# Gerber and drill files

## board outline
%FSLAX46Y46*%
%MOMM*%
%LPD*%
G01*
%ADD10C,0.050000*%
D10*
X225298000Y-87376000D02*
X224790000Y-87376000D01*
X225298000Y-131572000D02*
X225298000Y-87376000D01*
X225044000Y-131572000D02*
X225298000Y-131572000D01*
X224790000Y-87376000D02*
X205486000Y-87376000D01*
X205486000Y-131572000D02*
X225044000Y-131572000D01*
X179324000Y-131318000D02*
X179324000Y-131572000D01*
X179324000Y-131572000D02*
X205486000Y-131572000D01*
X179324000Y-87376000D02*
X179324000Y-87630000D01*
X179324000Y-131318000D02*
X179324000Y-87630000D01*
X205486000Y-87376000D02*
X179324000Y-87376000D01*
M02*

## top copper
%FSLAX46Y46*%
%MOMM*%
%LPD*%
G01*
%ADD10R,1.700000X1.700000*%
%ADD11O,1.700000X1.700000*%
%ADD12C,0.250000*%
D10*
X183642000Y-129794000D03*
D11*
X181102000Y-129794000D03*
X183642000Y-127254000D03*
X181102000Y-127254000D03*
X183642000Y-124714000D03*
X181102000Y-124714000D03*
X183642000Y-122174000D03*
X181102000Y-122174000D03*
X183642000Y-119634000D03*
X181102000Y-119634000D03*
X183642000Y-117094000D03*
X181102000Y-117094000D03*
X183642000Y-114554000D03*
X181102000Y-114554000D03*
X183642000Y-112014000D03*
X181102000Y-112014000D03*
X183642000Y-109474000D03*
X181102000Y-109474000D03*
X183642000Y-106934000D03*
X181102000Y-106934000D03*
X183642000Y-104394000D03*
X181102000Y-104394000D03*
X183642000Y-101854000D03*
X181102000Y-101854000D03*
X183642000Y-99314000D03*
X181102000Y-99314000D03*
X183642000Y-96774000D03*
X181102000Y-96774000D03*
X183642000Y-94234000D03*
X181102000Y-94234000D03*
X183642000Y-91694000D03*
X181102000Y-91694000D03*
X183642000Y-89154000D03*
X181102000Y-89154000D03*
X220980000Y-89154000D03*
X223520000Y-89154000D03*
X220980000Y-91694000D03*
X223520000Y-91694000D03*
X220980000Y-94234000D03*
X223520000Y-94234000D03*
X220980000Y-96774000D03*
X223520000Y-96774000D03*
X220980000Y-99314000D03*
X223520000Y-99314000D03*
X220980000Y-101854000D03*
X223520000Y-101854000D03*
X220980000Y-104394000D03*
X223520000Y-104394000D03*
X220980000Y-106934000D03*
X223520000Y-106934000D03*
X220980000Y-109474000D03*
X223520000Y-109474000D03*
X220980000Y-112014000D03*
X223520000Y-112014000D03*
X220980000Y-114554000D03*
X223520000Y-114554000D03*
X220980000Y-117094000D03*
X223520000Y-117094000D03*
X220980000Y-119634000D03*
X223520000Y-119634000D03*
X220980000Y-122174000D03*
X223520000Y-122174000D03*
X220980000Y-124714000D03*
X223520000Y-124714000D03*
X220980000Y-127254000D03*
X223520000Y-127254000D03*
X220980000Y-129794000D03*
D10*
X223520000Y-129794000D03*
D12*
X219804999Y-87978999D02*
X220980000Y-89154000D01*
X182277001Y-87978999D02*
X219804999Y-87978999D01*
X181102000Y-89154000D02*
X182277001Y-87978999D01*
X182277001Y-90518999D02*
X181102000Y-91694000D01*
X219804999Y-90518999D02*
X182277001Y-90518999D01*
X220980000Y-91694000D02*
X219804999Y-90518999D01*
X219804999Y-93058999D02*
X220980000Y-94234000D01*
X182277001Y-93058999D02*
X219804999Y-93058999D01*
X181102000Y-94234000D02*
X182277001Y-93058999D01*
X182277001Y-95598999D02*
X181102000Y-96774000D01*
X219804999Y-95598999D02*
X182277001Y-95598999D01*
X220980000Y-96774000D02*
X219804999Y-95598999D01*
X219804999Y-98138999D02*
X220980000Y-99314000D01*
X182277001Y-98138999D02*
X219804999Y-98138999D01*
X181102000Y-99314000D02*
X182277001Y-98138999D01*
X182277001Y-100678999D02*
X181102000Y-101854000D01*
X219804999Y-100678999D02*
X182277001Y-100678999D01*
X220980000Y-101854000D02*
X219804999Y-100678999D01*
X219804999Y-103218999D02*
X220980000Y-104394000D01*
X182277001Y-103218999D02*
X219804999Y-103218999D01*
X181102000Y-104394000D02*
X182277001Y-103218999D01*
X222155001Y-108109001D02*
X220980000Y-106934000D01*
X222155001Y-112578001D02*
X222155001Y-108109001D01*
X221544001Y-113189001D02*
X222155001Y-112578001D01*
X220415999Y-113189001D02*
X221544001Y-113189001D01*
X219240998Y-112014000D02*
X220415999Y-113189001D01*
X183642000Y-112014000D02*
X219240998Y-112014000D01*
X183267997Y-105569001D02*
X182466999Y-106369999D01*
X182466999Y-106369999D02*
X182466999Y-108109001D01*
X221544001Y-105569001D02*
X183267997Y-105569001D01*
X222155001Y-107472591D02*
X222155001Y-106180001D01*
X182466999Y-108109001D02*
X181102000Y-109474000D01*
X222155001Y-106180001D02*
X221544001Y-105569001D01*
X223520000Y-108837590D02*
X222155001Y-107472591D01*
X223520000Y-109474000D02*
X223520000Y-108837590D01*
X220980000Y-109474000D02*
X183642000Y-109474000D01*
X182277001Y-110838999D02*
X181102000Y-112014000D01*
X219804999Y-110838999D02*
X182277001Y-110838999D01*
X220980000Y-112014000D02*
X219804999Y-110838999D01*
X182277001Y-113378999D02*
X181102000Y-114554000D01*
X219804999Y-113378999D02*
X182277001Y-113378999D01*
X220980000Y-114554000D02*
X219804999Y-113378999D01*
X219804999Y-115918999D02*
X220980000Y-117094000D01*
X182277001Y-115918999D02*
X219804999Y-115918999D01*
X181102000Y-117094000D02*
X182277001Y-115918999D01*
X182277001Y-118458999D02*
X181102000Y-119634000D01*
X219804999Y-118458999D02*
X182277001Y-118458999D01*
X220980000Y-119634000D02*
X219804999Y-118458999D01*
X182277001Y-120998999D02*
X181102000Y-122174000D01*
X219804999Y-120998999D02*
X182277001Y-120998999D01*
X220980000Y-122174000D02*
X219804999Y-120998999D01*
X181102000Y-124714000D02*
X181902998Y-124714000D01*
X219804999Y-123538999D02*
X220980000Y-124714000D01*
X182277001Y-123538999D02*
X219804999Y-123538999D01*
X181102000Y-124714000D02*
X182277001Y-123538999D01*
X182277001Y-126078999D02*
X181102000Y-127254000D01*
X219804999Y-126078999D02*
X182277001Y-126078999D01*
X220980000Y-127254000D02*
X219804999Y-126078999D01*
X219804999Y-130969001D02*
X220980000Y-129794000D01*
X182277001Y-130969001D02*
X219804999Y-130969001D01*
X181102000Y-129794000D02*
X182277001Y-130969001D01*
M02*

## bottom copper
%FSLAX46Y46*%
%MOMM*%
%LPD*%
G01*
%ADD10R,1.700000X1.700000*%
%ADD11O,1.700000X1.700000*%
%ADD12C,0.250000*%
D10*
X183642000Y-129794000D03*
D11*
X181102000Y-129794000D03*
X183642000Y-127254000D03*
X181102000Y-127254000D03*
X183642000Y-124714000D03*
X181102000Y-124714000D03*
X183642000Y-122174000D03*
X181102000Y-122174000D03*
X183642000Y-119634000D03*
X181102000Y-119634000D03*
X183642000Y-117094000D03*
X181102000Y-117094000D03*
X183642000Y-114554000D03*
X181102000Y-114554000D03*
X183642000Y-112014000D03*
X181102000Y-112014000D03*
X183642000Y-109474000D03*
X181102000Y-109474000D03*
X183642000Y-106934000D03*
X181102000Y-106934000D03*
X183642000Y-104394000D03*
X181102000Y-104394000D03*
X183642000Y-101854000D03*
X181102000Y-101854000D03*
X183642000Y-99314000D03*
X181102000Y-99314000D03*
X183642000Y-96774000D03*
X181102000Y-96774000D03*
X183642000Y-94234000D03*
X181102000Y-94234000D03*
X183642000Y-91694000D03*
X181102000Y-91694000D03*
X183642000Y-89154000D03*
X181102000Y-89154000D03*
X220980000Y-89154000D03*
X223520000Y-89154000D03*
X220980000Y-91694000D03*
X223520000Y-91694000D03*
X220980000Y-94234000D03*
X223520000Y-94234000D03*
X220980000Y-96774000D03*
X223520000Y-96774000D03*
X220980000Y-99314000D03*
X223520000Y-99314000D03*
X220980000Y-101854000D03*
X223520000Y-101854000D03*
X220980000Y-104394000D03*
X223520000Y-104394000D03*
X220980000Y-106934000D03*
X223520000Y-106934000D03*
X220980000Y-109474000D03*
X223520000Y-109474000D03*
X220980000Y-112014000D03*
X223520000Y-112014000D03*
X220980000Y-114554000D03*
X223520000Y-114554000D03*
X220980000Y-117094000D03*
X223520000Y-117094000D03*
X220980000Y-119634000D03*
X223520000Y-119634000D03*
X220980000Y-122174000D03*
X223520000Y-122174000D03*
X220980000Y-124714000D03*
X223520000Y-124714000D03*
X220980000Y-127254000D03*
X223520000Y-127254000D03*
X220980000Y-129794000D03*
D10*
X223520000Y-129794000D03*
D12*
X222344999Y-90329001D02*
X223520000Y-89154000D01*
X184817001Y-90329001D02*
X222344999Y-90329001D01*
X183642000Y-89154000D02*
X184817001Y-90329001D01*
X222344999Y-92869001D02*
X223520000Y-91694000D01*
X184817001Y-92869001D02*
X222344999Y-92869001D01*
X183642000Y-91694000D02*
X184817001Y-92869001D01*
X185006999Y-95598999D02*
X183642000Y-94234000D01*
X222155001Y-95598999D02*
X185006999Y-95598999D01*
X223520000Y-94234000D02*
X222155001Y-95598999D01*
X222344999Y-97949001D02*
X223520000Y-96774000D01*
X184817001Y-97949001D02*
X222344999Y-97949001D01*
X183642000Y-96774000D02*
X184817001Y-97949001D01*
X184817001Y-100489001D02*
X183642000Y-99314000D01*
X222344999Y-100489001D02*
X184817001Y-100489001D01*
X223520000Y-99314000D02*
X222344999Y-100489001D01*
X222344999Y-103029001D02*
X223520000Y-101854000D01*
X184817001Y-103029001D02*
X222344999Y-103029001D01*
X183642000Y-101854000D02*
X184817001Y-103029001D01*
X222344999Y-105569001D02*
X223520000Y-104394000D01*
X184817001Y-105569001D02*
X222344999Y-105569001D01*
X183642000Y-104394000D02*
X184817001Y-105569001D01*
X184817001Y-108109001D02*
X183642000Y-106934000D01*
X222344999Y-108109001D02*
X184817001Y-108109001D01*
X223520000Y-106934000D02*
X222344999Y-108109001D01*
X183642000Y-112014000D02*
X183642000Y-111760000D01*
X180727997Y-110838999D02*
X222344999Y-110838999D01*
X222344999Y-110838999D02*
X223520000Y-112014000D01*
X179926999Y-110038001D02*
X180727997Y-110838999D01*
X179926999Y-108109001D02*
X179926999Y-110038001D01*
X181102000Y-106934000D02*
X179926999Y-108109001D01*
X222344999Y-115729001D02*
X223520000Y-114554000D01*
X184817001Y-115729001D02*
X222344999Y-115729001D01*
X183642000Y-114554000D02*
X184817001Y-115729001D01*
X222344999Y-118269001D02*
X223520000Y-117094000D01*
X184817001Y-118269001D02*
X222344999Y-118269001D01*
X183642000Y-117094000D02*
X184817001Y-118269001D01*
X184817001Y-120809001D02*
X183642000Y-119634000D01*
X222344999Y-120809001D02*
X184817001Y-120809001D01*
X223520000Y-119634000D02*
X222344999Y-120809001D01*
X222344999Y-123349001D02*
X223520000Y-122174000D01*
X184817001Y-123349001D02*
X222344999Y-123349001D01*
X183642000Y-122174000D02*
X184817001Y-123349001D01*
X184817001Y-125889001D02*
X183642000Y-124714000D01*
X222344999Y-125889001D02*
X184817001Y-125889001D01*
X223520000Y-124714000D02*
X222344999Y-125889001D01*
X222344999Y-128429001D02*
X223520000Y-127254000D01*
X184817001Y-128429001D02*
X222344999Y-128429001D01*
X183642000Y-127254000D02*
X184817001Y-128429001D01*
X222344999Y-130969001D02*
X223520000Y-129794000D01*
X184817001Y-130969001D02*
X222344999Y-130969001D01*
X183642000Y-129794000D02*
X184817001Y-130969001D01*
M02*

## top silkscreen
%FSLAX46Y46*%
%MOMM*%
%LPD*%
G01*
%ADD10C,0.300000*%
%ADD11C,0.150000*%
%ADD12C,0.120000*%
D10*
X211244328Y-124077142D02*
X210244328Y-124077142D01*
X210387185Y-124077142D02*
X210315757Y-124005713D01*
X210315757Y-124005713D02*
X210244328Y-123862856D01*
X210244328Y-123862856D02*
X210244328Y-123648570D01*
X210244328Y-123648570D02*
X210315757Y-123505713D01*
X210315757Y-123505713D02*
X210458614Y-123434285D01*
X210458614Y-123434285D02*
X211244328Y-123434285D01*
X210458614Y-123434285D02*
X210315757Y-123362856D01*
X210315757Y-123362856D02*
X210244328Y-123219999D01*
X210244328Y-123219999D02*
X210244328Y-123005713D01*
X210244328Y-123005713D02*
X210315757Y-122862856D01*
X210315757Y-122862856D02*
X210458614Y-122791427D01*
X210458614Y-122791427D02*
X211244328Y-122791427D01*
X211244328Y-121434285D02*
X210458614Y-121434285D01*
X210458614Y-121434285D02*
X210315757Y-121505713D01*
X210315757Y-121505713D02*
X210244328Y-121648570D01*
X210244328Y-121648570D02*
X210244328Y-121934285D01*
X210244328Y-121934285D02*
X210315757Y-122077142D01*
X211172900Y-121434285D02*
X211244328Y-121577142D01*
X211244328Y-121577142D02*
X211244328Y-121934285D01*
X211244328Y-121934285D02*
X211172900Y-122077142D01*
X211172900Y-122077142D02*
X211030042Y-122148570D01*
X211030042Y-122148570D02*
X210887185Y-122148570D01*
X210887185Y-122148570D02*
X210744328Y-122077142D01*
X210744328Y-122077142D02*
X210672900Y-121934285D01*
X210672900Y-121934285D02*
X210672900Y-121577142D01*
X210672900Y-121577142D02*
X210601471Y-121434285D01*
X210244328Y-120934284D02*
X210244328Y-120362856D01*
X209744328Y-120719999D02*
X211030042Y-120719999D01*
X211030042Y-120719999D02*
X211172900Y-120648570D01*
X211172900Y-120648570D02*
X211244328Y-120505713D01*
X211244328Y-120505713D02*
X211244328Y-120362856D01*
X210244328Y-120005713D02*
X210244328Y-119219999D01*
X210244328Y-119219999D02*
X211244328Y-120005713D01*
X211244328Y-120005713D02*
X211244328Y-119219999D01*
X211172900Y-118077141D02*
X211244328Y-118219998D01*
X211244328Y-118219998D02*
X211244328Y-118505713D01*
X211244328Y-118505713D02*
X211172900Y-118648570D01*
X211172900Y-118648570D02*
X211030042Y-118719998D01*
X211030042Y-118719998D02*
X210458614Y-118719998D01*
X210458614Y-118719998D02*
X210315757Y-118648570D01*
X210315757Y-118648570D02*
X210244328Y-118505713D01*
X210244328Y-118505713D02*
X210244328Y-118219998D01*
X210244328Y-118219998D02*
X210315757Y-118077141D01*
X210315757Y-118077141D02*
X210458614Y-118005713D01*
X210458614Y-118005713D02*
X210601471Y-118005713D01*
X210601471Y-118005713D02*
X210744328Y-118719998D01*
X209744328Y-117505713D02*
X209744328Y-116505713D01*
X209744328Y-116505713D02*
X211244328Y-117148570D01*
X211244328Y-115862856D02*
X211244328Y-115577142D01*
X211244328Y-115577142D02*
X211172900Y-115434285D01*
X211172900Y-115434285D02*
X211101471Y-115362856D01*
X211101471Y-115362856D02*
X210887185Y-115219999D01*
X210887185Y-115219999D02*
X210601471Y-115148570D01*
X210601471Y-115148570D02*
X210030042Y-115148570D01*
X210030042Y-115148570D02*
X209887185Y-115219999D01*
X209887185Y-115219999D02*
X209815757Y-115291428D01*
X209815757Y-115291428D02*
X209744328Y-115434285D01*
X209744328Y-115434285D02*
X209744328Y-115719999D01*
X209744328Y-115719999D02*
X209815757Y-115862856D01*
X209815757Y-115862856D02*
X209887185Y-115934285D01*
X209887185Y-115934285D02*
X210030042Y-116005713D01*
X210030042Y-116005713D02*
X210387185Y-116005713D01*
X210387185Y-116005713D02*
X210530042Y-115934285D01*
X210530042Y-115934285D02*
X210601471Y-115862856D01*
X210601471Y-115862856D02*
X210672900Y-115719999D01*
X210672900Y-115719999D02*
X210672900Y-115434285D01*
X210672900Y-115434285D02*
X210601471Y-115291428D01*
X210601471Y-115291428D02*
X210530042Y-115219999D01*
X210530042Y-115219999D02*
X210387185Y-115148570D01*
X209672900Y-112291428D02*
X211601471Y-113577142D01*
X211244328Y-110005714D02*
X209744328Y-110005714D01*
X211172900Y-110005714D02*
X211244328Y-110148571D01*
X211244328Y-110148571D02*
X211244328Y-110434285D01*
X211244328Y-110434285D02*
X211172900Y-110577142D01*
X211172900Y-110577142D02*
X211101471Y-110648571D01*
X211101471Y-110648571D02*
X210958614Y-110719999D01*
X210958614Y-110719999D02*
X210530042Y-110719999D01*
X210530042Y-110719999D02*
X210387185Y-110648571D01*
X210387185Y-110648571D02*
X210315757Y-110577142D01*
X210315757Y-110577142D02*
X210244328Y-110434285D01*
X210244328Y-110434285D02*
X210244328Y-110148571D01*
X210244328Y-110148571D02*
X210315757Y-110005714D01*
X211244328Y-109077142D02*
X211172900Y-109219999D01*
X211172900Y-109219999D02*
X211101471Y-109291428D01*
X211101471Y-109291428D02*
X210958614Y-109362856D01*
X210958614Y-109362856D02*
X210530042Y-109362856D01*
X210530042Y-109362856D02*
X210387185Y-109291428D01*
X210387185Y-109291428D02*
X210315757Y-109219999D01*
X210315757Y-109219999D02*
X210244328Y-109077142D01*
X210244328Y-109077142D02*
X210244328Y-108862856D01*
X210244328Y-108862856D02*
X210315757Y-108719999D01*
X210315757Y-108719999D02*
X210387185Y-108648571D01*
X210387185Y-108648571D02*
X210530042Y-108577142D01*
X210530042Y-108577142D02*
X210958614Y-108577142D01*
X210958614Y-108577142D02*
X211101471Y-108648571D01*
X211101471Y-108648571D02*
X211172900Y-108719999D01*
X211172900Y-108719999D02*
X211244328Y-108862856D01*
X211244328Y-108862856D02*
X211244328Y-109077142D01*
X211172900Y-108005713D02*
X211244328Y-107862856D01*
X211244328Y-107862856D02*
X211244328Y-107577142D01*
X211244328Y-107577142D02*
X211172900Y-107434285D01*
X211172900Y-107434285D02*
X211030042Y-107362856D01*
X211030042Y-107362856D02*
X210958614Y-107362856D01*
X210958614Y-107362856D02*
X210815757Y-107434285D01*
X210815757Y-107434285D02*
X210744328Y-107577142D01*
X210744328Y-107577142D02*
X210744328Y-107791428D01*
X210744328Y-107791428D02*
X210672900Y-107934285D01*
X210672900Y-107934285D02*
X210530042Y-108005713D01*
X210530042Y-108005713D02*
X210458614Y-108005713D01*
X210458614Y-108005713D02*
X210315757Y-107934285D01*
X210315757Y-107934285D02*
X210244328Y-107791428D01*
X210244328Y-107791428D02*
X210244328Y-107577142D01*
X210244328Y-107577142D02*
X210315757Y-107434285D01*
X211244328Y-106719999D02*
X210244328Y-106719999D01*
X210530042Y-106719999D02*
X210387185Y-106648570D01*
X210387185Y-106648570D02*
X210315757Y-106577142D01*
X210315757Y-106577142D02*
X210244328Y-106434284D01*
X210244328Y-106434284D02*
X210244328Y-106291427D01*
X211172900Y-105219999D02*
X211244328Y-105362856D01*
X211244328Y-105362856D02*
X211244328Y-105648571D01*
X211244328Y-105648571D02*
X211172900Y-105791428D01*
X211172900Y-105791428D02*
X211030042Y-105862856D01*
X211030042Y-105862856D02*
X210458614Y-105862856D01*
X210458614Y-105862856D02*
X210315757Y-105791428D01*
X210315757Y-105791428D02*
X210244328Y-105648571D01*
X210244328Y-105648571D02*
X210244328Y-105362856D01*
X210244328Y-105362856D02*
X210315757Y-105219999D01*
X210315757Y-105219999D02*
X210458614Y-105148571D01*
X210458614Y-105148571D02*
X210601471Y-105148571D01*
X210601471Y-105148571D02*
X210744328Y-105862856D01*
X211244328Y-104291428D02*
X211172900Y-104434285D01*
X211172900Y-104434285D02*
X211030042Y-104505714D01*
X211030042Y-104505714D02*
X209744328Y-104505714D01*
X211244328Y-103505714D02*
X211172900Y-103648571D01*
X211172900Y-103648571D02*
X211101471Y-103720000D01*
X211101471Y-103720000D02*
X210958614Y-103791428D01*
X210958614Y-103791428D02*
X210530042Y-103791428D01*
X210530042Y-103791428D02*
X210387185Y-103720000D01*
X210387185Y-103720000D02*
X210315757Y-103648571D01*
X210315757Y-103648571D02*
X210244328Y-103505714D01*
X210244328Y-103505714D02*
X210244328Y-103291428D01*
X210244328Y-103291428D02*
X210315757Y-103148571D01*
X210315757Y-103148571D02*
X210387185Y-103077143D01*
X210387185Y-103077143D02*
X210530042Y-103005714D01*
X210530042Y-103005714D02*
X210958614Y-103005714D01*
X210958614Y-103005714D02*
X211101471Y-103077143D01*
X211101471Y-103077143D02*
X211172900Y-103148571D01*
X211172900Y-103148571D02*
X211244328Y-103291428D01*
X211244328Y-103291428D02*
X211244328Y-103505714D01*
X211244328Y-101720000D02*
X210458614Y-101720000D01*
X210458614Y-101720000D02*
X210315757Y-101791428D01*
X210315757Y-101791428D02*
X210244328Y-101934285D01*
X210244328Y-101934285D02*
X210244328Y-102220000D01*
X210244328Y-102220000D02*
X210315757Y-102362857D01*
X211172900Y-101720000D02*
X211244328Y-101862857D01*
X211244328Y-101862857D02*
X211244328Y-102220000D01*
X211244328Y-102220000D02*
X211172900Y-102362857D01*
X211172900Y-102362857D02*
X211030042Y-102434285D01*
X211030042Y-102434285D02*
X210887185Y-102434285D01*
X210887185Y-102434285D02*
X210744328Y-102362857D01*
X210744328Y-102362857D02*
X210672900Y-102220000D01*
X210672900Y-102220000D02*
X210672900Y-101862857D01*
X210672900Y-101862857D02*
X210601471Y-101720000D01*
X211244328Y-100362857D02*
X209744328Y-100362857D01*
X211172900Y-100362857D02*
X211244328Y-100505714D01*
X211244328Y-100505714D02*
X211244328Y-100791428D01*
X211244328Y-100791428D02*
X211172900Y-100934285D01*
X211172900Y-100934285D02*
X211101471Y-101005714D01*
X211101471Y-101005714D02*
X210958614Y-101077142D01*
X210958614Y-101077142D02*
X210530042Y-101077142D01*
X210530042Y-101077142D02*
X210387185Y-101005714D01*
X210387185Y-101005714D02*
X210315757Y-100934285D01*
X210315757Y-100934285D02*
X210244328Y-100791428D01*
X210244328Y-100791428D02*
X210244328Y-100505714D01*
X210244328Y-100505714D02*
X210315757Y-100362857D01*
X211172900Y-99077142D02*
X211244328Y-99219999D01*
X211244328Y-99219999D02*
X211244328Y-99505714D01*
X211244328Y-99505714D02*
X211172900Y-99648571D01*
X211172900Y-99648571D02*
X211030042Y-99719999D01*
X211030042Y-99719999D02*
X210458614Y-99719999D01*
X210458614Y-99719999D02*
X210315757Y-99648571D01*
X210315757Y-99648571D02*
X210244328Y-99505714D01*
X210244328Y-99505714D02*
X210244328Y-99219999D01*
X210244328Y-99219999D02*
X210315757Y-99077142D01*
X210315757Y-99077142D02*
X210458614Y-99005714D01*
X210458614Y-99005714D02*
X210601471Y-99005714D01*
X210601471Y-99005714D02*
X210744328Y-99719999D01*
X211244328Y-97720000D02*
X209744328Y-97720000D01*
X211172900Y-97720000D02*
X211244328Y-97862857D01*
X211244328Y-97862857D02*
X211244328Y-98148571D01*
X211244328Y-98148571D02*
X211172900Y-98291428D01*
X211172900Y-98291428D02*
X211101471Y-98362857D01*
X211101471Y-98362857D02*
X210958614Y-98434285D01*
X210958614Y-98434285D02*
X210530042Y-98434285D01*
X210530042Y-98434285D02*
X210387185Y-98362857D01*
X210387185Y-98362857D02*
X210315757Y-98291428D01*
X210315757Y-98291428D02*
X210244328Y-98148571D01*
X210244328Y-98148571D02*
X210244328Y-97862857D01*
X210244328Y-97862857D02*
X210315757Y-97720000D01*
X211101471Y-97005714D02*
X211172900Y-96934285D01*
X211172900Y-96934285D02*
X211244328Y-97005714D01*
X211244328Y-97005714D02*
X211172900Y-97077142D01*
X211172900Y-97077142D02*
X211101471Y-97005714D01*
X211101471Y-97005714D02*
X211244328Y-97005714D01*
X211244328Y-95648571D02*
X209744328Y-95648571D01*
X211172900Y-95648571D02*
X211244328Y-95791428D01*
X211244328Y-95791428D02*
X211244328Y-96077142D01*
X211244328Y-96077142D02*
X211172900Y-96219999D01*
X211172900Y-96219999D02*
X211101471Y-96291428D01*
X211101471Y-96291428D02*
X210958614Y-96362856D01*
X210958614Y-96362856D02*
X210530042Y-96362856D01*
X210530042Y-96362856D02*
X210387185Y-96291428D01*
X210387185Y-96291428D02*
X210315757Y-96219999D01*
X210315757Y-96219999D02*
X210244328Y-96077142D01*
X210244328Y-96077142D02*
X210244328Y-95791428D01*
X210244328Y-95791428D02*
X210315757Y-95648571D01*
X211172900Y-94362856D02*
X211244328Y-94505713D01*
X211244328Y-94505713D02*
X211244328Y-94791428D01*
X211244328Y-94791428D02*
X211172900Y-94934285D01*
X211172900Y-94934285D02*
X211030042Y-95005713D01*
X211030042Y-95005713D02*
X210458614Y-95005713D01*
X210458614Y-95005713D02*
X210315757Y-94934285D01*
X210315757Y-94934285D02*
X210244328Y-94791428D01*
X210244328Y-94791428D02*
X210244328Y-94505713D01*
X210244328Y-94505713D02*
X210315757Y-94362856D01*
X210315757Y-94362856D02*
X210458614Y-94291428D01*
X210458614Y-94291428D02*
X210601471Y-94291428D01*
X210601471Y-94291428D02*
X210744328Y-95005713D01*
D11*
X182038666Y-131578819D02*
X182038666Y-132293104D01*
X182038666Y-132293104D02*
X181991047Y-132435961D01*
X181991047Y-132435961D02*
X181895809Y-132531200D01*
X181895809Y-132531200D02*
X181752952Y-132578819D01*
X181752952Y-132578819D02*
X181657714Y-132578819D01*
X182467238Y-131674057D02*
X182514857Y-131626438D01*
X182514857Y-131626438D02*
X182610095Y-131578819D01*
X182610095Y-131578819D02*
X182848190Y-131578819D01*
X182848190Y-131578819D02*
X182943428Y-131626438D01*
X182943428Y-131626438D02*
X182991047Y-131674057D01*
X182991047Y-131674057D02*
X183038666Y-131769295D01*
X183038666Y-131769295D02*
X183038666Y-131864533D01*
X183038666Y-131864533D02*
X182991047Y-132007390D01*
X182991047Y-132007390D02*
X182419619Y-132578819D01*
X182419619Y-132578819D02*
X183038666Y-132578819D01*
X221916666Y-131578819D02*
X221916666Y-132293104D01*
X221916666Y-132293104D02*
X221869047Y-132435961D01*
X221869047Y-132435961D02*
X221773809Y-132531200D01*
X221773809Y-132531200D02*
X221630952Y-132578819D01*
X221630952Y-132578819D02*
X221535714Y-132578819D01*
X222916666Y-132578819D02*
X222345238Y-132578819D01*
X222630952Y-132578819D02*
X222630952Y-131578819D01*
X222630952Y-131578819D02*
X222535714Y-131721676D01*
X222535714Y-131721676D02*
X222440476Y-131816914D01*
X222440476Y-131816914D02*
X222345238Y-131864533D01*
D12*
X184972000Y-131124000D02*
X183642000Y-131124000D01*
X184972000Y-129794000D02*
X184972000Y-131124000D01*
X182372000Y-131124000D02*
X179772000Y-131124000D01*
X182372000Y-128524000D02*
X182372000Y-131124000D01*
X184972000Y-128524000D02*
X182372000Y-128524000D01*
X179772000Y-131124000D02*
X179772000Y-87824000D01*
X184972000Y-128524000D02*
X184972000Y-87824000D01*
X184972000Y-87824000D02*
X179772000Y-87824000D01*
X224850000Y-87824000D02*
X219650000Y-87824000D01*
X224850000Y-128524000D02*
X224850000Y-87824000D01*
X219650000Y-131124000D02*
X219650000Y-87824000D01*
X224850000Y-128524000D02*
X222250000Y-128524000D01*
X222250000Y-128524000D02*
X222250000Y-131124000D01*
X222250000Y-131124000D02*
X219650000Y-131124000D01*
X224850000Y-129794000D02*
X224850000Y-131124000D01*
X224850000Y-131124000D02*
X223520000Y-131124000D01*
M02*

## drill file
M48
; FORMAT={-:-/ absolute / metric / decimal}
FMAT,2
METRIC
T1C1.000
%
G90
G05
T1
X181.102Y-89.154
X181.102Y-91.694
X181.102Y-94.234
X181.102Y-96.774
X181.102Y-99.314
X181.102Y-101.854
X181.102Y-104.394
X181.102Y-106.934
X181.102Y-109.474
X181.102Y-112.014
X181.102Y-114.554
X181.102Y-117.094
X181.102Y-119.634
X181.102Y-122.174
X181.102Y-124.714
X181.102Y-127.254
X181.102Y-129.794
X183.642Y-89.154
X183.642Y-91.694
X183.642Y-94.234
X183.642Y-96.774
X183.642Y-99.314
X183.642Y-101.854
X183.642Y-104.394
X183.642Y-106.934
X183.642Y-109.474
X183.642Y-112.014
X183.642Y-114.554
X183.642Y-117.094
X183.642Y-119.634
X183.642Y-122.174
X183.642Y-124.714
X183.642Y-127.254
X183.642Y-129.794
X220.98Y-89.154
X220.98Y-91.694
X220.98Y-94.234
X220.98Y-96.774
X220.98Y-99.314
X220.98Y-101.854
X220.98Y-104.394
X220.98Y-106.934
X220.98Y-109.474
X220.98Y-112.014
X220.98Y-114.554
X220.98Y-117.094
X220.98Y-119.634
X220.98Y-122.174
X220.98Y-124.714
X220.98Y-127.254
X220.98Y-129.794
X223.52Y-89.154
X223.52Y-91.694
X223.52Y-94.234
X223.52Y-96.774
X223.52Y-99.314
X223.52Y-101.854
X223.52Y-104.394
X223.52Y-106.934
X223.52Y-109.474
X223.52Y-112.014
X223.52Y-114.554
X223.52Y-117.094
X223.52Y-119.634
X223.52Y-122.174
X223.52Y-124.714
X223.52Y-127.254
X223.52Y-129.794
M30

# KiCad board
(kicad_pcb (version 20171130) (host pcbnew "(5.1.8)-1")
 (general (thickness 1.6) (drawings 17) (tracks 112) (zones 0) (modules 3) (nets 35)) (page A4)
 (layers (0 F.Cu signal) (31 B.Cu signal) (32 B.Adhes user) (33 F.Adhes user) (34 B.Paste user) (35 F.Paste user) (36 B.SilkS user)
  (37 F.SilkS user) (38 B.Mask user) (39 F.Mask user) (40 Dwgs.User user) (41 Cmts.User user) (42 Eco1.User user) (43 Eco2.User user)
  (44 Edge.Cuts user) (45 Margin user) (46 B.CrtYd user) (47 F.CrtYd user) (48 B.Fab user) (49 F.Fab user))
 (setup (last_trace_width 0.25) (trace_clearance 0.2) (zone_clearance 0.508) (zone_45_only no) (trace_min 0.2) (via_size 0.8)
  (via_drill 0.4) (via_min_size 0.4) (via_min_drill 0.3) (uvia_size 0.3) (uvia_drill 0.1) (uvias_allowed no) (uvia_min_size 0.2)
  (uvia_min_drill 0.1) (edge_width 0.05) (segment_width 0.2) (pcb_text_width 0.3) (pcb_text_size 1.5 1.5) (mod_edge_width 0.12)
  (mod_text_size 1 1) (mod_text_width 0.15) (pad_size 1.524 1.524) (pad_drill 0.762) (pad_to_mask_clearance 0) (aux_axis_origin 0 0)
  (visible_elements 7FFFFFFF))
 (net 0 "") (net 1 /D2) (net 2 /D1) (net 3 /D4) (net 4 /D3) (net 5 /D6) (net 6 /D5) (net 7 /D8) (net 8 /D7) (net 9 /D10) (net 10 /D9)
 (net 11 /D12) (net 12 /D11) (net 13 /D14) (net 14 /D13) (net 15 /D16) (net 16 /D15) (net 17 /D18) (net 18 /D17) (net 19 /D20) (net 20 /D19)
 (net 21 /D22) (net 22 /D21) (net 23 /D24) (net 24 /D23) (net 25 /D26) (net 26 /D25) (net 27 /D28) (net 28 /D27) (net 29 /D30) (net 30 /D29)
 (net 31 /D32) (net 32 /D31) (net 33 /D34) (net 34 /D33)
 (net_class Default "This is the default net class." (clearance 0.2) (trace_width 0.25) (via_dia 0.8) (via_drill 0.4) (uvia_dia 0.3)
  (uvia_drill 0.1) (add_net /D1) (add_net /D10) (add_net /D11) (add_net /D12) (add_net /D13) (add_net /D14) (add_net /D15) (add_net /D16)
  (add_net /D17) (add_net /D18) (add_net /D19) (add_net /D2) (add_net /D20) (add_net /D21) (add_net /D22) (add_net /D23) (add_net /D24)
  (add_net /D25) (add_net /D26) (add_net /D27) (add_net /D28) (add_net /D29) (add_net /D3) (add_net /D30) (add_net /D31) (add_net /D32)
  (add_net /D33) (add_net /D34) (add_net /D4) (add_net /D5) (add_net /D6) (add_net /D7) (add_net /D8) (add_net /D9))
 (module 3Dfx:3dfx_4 (layer B.Cu) (at 205.994 109.22 270)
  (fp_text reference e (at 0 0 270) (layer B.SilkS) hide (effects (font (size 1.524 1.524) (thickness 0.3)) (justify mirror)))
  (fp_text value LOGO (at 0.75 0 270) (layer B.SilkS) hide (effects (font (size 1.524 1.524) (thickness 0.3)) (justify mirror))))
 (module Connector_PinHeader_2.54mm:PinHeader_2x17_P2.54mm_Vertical (layer F.Cu) (at 183.642 129.794 180)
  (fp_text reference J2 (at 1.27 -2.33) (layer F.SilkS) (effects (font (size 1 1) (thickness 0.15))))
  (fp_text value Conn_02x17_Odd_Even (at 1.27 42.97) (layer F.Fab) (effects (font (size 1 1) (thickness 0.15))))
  (fp_line (start -1.33 -1.33) (end 0 -1.33) (layer F.SilkS) (width 0.12))
  (fp_line (start -1.33 0) (end -1.33 -1.33) (layer F.SilkS) (width 0.12))
  (fp_line (start 1.27 -1.33) (end 3.87 -1.33) (layer F.SilkS) (width 0.12))
  (fp_line (start 1.27 1.27) (end 1.27 -1.33) (layer F.SilkS) (width 0.12))
  (fp_line (start -1.33 1.27) (end 1.27 1.27) (layer F.SilkS) (width 0.12))
  (fp_line (start 3.87 -1.33) (end 3.87 41.97) (layer F.SilkS) (width 0.12))
  (fp_line (start -1.33 1.27) (end -1.33 41.97) (layer F.SilkS) (width 0.12))
  (fp_line (start -1.33 41.97) (end 3.87 41.97) (layer F.SilkS) (width 0.12))
  (pad 1 thru_hole rect (at 0 0 180) (size 1.7 1.7) (drill 1) (layers *.Cu *.Mask) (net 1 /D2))
  (pad 2 thru_hole oval (at 2.54 0 180) (size 1.7 1.7) (drill 1) (layers *.Cu *.Mask) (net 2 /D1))
  (pad 3 thru_hole oval (at 0 2.54 180) (size 1.7 1.7) (drill 1) (layers *.Cu *.Mask) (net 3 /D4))
  (pad 4 thru_hole oval (at 2.54 2.54 180) (size 1.7 1.7) (drill 1) (layers *.Cu *.Mask) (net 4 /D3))
  (pad 5 thru_hole oval (at 0 5.08 180) (size 1.7 1.7) (drill 1) (layers *.Cu *.Mask) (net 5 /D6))
  (pad 6 thru_hole oval (at 2.54 5.08 180) (size 1.7 1.7) (drill 1) (layers *.Cu *.Mask) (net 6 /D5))
  (pad 7 thru_hole oval (at 0 7.62 180) (size 1.7 1.7) (drill 1) (layers *.Cu *.Mask) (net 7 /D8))
  (pad 8 thru_hole oval (at 2.54 7.62 180) (size 1.7 1.7) (drill 1) (layers *.Cu *.Mask) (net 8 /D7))
  (pad 9 thru_hole oval (at 0 10.16 180) (size 1.7 1.7) (drill 1) (layers *.Cu *.Mask) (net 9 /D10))
  (pad 10 thru_hole oval (at 2.54 10.16 180) (size 1.7 1.7) (drill 1) (layers *.Cu *.Mask) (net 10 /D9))
  (pad 11 thru_hole oval (at 0 12.7 180) (size 1.7 1.7) (drill 1) (layers *.Cu *.Mask) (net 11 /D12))
  (pad 12 thru_hole oval (at 2.54 12.7 180) (size 1.7 1.7) (drill 1) (layers *.Cu *.Mask) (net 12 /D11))
  (pad 13 thru_hole oval (at 0 15.24 180) (size 1.7 1.7) (drill 1) (layers *.Cu *.Mask) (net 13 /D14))
  (pad 14 thru_hole oval (at 2.54 15.24 180) (size 1.7 1.7) (drill 1) (layers *.Cu *.Mask) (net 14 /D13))
  (pad 15 thru_hole oval (at 0 17.78 180) (size 1.7 1.7) (drill 1) (layers *.Cu *.Mask) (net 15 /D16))
  (pad 16 thru_hole oval (at 2.54 17.78 180) (size 1.7 1.7) (drill 1) (layers *.Cu *.Mask) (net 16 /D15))
  (pad 17 thru_hole oval (at 0 20.32 180) (size 1.7 1.7) (drill 1) (layers *.Cu *.Mask) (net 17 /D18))
  (pad 18 thru_hole oval (at 2.54 20.32 180) (size 1.7 1.7) (drill 1) (layers *.Cu *.Mask) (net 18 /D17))
  (pad 19 thru_hole oval (at 0 22.86 180) (size 1.7 1.7) (drill 1) (layers *.Cu *.Mask) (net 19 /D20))
  (pad 20 thru_hole oval (at 2.54 22.86 180) (size 1.7 1.7) (drill 1) (layers *.Cu *.Mask) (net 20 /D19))
  (pad 21 thru_hole oval (at 0 25.4 180) (size 1.7 1.7) (drill 1) (layers *.Cu *.Mask) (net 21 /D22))
  (pad 22 thru_hole oval (at 2.54 25.4 180) (size 1.7 1.7) (drill 1) (layers *.Cu *.Mask) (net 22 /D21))
  (pad 23 thru_hole oval (at 0 27.94 180) (size 1.7 1.7) (drill 1) (layers *.Cu *.Mask) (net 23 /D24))
  (pad 24 thru_hole oval (at 2.54 27.94 180) (size 1.7 1.7) (drill 1) (layers *.Cu *.Mask) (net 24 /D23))
  (pad 25 thru_hole oval (at 0 30.48 180) (size 1.7 1.7) (drill 1) (layers *.Cu *.Mask) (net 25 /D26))
  (pad 26 thru_hole oval (at 2.54 30.48 180) (size 1.7 1.7) (drill 1) (layers *.Cu *.Mask) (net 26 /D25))
  (pad 27 thru_hole oval (at 0 33.02 180) (size 1.7 1.7) (drill 1) (layers *.Cu *.Mask) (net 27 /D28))
  (pad 28 thru_hole oval (at 2.54 33.02 180) (size 1.7 1.7) (drill 1) (layers *.Cu *.Mask) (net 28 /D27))
  (pad 29 thru_hole oval (at 0 35.56 180) (size 1.7 1.7) (drill 1) (layers *.Cu *.Mask) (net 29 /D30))
  (pad 30 thru_hole oval (at 2.54 35.56 180) (size 1.7 1.7) (drill 1) (layers *.Cu *.Mask) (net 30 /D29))
  (pad 31 thru_hole oval (at 0 38.1 180) (size 1.7 1.7) (drill 1) (layers *.Cu *.Mask) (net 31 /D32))
  (pad 32 thru_hole oval (at 2.54 38.1 180) (size 1.7 1.7) (drill 1) (layers *.Cu *.Mask) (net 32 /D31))
  (pad 33 thru_hole oval (at 0 40.64 180) (size 1.7 1.7) (drill 1) (layers *.Cu *.Mask) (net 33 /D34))
  (pad 34 thru_hole oval (at 2.54 40.64 180) (size 1.7 1.7) (drill 1) (layers *.Cu *.Mask) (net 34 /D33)))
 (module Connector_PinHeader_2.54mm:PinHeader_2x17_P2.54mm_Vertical (layer F.Cu) (at 223.52 129.794 180)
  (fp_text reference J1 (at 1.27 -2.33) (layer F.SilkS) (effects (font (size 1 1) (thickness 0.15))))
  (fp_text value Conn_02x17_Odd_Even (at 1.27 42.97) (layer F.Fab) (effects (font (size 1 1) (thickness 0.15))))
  (fp_line (start -1.33 41.97) (end 3.87 41.97) (layer F.SilkS) (width 0.12))
  (fp_line (start -1.33 1.27) (end -1.33 41.97) (layer F.SilkS) (width 0.12))
  (fp_line (start 3.87 -1.33) (end 3.87 41.97) (layer F.SilkS) (width 0.12))
  (fp_line (start -1.33 1.27) (end 1.27 1.27) (layer F.SilkS) (width 0.12))
  (fp_line (start 1.27 1.27) (end 1.27 -1.33) (layer F.SilkS) (width 0.12))
  (fp_line (start 1.27 -1.33) (end 3.87 -1.33) (layer F.SilkS) (width 0.12))
  (fp_line (start -1.33 0) (end -1.33 -1.33) (layer F.SilkS) (width 0.12))
  (fp_line (start -1.33 -1.33) (end 0 -1.33) (layer F.SilkS) (width 0.12))
  (pad 34 thru_hole oval (at 2.54 40.64 180) (size 1.7 1.7) (drill 1) (layers *.Cu *.Mask) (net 34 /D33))
  (pad 33 thru_hole oval (at 0 40.64 180) (size 1.7 1.7) (drill 1) (layers *.Cu *.Mask) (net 33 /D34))
  (pad 32 thru_hole oval (at 2.54 38.1 180) (size 1.7 1.7) (drill 1) (layers *.Cu *.Mask) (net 32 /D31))
  (pad 31 thru_hole oval (at 0 38.1 180) (size 1.7 1.7) (drill 1) (layers *.Cu *.Mask) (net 31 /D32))
  (pad 30 thru_hole oval (at 2.54 35.56 180) (size 1.7 1.7) (drill 1) (layers *.Cu *.Mask) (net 30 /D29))
  (pad 29 thru_hole oval (at 0 35.56 180) (size 1.7 1.7) (drill 1) (layers *.Cu *.Mask) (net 29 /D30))
  (pad 28 thru_hole oval (at 2.54 33.02 180) (size 1.7 1.7) (drill 1) (layers *.Cu *.Mask) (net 28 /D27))
  (pad 27 thru_hole oval (at 0 33.02 180) (size 1.7 1.7) (drill 1) (layers *.Cu *.Mask) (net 27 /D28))
  (pad 26 thru_hole oval (at 2.54 30.48 180) (size 1.7 1.7) (drill 1) (layers *.Cu *.Mask) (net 26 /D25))
  (pad 25 thru_hole oval (at 0 30.48 180) (size 1.7 1.7) (drill 1) (layers *.Cu *.Mask) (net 25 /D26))
  (pad 24 thru_hole oval (at 2.54 27.94 180) (size 1.7 1.7) (drill 1) (layers *.Cu *.Mask) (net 24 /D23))
  (pad 23 thru_hole oval (at 0 27.94 180) (size 1.7 1.7) (drill 1) (layers *.Cu *.Mask) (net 23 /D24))
  (pad 22 thru_hole oval (at 2.54 25.4 180) (size 1.7 1.7) (drill 1) (layers *.Cu *.Mask) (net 22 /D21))
  (pad 21 thru_hole oval (at 0 25.4 180) (size 1.7 1.7) (drill 1) (layers *.Cu *.Mask) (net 21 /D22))
  (pad 20 thru_hole oval (at 2.54 22.86 180) (size 1.7 1.7) (drill 1) (layers *.Cu *.Mask) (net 15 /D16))
  (pad 19 thru_hole oval (at 0 22.86 180) (size 1.7 1.7) (drill 1) (layers *.Cu *.Mask) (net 19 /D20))
  (pad 18 thru_hole oval (at 2.54 20.32 180) (size 1.7 1.7) (drill 1) (layers *.Cu *.Mask) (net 17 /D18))
  (pad 17 thru_hole oval (at 0 20.32 180) (size 1.7 1.7) (drill 1) (layers *.Cu *.Mask) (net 18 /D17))
  (pad 16 thru_hole oval (at 2.54 17.78 180) (size 1.7 1.7) (drill 1) (layers *.Cu *.Mask) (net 16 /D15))
  (pad 15 thru_hole oval (at 0 17.78 180) (size 1.7 1.7) (drill 1) (layers *.Cu *.Mask) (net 20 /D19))
  (pad 14 thru_hole oval (at 2.54 15.24 180) (size 1.7 1.7) (drill 1) (layers *.Cu *.Mask) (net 14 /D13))
  (pad 13 thru_hole oval (at 0 15.24 180) (size 1.7 1.7) (drill 1) (layers *.Cu *.Mask) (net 13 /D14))
  (pad 12 thru_hole oval (at 2.54 12.7 180) (size 1.7 1.7) (drill 1) (layers *.Cu *.Mask) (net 12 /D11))
  (pad 11 thru_hole oval (at 0 12.7 180) (size 1.7 1.7) (drill 1) (layers *.Cu *.Mask) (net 11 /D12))
  (pad 10 thru_hole oval (at 2.54 10.16 180) (size 1.7 1.7) (drill 1) (layers *.Cu *.Mask) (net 10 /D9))
  (pad 9 thru_hole oval (at 0 10.16 180) (size 1.7 1.7) (drill 1) (layers *.Cu *.Mask) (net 9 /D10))
  (pad 8 thru_hole oval (at 2.54 7.62 180) (size 1.7 1.7) (drill 1) (layers *.Cu *.Mask) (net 8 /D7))
  (pad 7 thru_hole oval (at 0 7.62 180) (size 1.7 1.7) (drill 1) (layers *.Cu *.Mask) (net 7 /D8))
  (pad 6 thru_hole oval (at 2.54 5.08 180) (size 1.7 1.7) (drill 1) (layers *.Cu *.Mask) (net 6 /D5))
  (pad 5 thru_hole oval (at 0 5.08 180) (size 1.7 1.7) (drill 1) (layers *.Cu *.Mask) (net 5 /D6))
  (pad 4 thru_hole oval (at 2.54 2.54 180) (size 1.7 1.7) (drill 1) (layers *.Cu *.Mask) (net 4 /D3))
  (pad 3 thru_hole oval (at 0 2.54 180) (size 1.7 1.7) (drill 1) (layers *.Cu *.Mask) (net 3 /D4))
  (pad 2 thru_hole oval (at 2.54 0 180) (size 1.7 1.7) (drill 1) (layers *.Cu *.Mask) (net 2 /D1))
  (pad 1 thru_hole rect (at 0 0 180) (size 1.7 1.7) (drill 1) (layers *.Cu *.Mask) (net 1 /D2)))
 (gr_line (start 225.298 87.376) (end 224.79 87.376) (layer Edge.Cuts) (width 0.05))
 (gr_line (start 225.298 131.572) (end 225.298 87.376) (layer Edge.Cuts) (width 0.05))
 (gr_line (start 225.044 131.572) (end 225.298 131.572) (layer Edge.Cuts) (width 0.05))
 (gr_line (start 224.79 87.376) (end 205.486 87.376) (layer Edge.Cuts) (width 0.05))
 (gr_line (start 205.486 131.572) (end 225.044 131.572) (layer Edge.Cuts) (width 0.05))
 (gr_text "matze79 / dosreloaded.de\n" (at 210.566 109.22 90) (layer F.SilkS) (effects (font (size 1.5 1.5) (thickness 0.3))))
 (gr_line (start 179.324 131.318) (end 179.324 131.572) (layer Edge.Cuts) (width 0.05))
 (gr_line (start 179.324 131.572) (end 205.486 131.572) (layer Edge.Cuts) (width 0.05))
 (gr_line (start 179.324 87.376) (end 179.324 87.63) (layer Edge.Cuts) (width 0.05))
 (gr_line (start 179.324 131.318) (end 179.324 87.63) (layer Edge.Cuts) (width 0.05))
 (gr_line (start 205.486 87.376) (end 179.324 87.376) (layer Edge.Cuts) (width 0.05))
 (segment (start 222.344999 90.329001) (end 223.52 89.154) (width 0.25) (layer B.Cu) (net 33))
 (segment (start 184.817001 90.329001) (end 222.344999 90.329001) (width 0.25) (layer B.Cu) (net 33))
 (segment (start 183.642 89.154) (end 184.817001 90.329001) (width 0.25) (layer B.Cu) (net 33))
 (segment (start 219.804999 87.978999) (end 220.98 89.154) (width 0.25) (layer F.Cu) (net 34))
 (segment (start 182.277001 87.978999) (end 219.804999 87.978999) (width 0.25) (layer F.Cu) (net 34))
 (segment (start 181.102 89.154) (end 182.277001 87.978999) (width 0.25) (layer F.Cu) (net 34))
 (segment (start 222.344999 92.869001) (end 223.52 91.694) (width 0.25) (layer B.Cu) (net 31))
 (segment (start 184.817001 92.869001) (end 222.344999 92.869001) (width 0.25) (layer B.Cu) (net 31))
 (segment (start 183.642 91.694) (end 184.817001 92.869001) (width 0.25) (layer B.Cu) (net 31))
 (segment (start 182.277001 90.518999) (end 181.102 91.694) (width 0.25) (layer F.Cu) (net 32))
 (segment (start 219.804999 90.518999) (end 182.277001 90.518999) (width 0.25) (layer F.Cu) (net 32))
 (segment (start 220.98 91.694) (end 219.804999 90.518999) (width 0.25) (layer F.Cu) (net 32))
 (segment (start 185.006999 95.598999) (end 183.642 94.234) (width 0.25) (layer B.Cu) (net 29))
 (segment (start 222.155001 95.598999) (end 185.006999 95.598999) (width 0.25) (layer B.Cu) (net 29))
 (segment (start 223.52 94.234) (end 222.155001 95.598999) (width 0.25) (layer B.Cu) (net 29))
 (segment (start 219.804999 93.058999) (end 220.98 94.234) (width 0.25) (layer F.Cu) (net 30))
 (segment (start 182.277001 93.058999) (end 219.804999 93.058999) (width 0.25) (layer F.Cu) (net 30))
 (segment (start 181.102 94.234) (end 182.277001 93.058999) (width 0.25) (layer F.Cu) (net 30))
 (segment (start 222.344999 97.949001) (end 223.52 96.774) (width 0.25) (layer B.Cu) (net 27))
 (segment (start 184.817001 97.949001) (end 222.344999 97.949001) (width 0.25) (layer B.Cu) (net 27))
 (segment (start 183.642 96.774) (end 184.817001 97.949001) (width 0.25) (layer B.Cu) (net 27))
 (segment (start 182.277001 95.598999) (end 181.102 96.774) (width 0.25) (layer F.Cu) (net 28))
 (segment (start 219.804999 95.598999) (end 182.277001 95.598999) (width 0.25) (layer F.Cu) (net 28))
 (segment (start 220.98 96.774) (end 219.804999 95.598999) (width 0.25) (layer F.Cu) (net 28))
 (segment (start 184.817001 100.489001) (end 183.642 99.314) (width 0.25) (layer B.Cu) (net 25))
 (segment (start 222.344999 100.489001) (end 184.817001 100.489001) (width 0.25) (layer B.Cu) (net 25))
 (segment (start 223.52 99.314) (end 222.344999 100.489001) (width 0.25) (layer B.Cu) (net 25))
 (segment (start 219.804999 98.138999) (end 220.98 99.314) (width 0.25) (layer F.Cu) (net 26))
 (segment (start 182.277001 98.138999) (end 219.804999 98.138999) (width 0.25) (layer F.Cu) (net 26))
 (segment (start 181.102 99.314) (end 182.277001 98.138999) (width 0.25) (layer F.Cu) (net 26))
 (segment (start 222.344999 103.029001) (end 223.52 101.854) (width 0.25) (layer B.Cu) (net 23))
 (segment (start 184.817001 103.029001) (end 222.344999 103.029001) (width 0.25) (layer B.Cu) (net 23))
 (segment (start 183.642 101.854) (end 184.817001 103.029001) (width 0.25) (layer B.Cu) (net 23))
 (segment (start 182.277001 100.678999) (end 181.102 101.854) (width 0.25) (layer F.Cu) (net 24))
 (segment (start 219.804999 100.678999) (end 182.277001 100.678999) (width 0.25) (layer F.Cu) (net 24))
 (segment (start 220.98 101.854) (end 219.804999 100.678999) (width 0.25) (layer F.Cu) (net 24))
 (segment (start 222.344999 105.569001) (end 223.52 104.394) (width 0.25) (layer B.Cu) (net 21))
 (segment (start 184.817001 105.569001) (end 222.344999 105.569001) (width 0.25) (layer B.Cu) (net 21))
 (segment (start 183.642 104.394) (end 184.817001 105.569001) (width 0.25) (layer B.Cu) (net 21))
 (segment (start 219.804999 103.218999) (end 220.98 104.394) (width 0.25) (layer F.Cu) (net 22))
 (segment (start 182.277001 103.218999) (end 219.804999 103.218999) (width 0.25) (layer F.Cu) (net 22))
 (segment (start 181.102 104.394) (end 182.277001 103.218999) (width 0.25) (layer F.Cu) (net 22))
 (segment (start 184.817001 108.109001) (end 183.642 106.934) (width 0.25) (layer B.Cu) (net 19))
 (segment (start 222.344999 108.109001) (end 184.817001 108.109001) (width 0.25) (layer B.Cu) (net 19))
 (segment (start 223.52 106.934) (end 222.344999 108.109001) (width 0.25) (layer B.Cu) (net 19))
 (segment (start 183.642 112.014) (end 183.642 111.76) (width 0.25) (layer B.Cu) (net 15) (status 30))
 (segment (start 222.155001 108.109001) (end 220.98 106.934) (width 0.25) (layer F.Cu) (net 15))
 (segment (start 222.155001 112.578001) (end 222.155001 108.109001) (width 0.25) (layer F.Cu) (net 15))
 (segment (start 221.544001 113.189001) (end 222.155001 112.578001) (width 0.25) (layer F.Cu) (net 15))
 (segment (start 220.415999 113.189001) (end 221.544001 113.189001) (width 0.25) (layer F.Cu) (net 15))
 (segment (start 219.240998 112.014) (end 220.415999 113.189001) (width 0.25) (layer F.Cu) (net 15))
 (segment (start 183.642 112.014) (end 219.240998 112.014) (width 0.25) (layer F.Cu) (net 15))
 (segment (start 183.267997 105.569001) (end 182.466999 106.369999) (width 0.25) (layer F.Cu) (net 18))
 (segment (start 182.466999 106.369999) (end 182.466999 108.109001) (width 0.25) (layer F.Cu) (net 18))
 (segment (start 221.544001 105.569001) (end 183.267997 105.569001) (width 0.25) (layer F.Cu) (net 18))
 (segment (start 222.155001 107.472591) (end 222.155001 106.180001) (width 0.25) (layer F.Cu) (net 18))
 (segment (start 182.466999 108.109001) (end 181.102 109.474) (width 0.25) (layer F.Cu) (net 18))
 (segment (start 222.155001 106.180001) (end 221.544001 105.569001) (width 0.25) (layer F.Cu) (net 18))
 (segment (start 223.52 108.83759) (end 222.155001 107.472591) (width 0.25) (layer F.Cu) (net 18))
 (segment (start 223.52 109.474) (end 223.52 108.83759) (width 0.25) (layer F.Cu) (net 18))
 (segment (start 220.98 109.474) (end 183.642 109.474) (width 0.25) (layer F.Cu) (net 17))
 (segment (start 180.727997 110.838999) (end 222.344999 110.838999) (width 0.25) (layer B.Cu) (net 20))
 (segment (start 222.344999 110.838999) (end 223.52 112.014) (width 0.25) (layer B.Cu) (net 20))
 (segment (start 179.926999 110.038001) (end 180.727997 110.838999) (width 0.25) (layer B.Cu) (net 20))
 (segment (start 179.926999 108.109001) (end 179.926999 110.038001) (width 0.25) (layer B.Cu) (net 20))
 (segment (start 181.102 106.934) (end 179.926999 108.109001) (width 0.25) (layer B.Cu) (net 20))
 (segment (start 182.277001 110.838999) (end 181.102 112.014) (width 0.25) (layer F.Cu) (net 16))
 (segment (start 219.804999 110.838999) (end 182.277001 110.838999) (width 0.25) (layer F.Cu) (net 16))
 (segment (start 220.98 112.014) (end 219.804999 110.838999) (width 0.25) (layer F.Cu) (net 16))
 (segment (start 222.344999 115.729001) (end 223.52 114.554) (width 0.25) (layer B.Cu) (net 13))
 (segment (start 184.817001 115.729001) (end 222.344999 115.729001) (width 0.25) (layer B.Cu) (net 13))
 (segment (start 183.642 114.554) (end 184.817001 115.729001) (width 0.25) (layer B.Cu) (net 13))
 (segment (start 182.277001 113.378999) (end 181.102 114.554) (width 0.25) (layer F.Cu) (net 14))
 (segment (start 219.804999 113.378999) (end 182.277001 113.378999) (width 0.25) (layer F.Cu) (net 14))
 (segment (start 220.98 114.554) (end 219.804999 113.378999) (width 0.25) (layer F.Cu) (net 14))
 (segment (start 222.344999 118.269001) (end 223.52 117.094) (width 0.25) (layer B.Cu) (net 11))
 (segment (start 184.817001 118.269001) (end 222.344999 118.269001) (width 0.25) (layer B.Cu) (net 11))
 (segment (start 183.642 117.094) (end 184.817001 118.269001) (width 0.25) (layer B.Cu) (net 11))
 (segment (start 219.804999 115.918999) (end 220.98 117.094) (width 0.25) (layer F.Cu) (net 12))
 (segment (start 182.277001 115.918999) (end 219.804999 115.918999) (width 0.25) (layer F.Cu) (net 12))
 (segment (start 181.102 117.094) (end 182.277001 115.918999) (width 0.25) (layer F.Cu) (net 12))
 (segment (start 184.817001 120.809001) (end 183.642 119.634) (width 0.25) (layer B.Cu) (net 9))
 (segment (start 222.344999 120.809001) (end 184.817001 120.809001) (width 0.25) (layer B.Cu) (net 9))
 (segment (start 223.52 119.634) (end 222.344999 120.809001) (width 0.25) (layer B.Cu) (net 9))
 (segment (start 182.277001 118.458999) (end 181.102 119.634) (width 0.25) (layer F.Cu) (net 10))
 (segment (start 219.804999 118.458999) (end 182.277001 118.458999) (width 0.25) (layer F.Cu) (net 10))
 (segment (start 220.98 119.634) (end 219.804999 118.458999) (width 0.25) (layer F.Cu) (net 10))
 (segment (start 222.344999 123.349001) (end 223.52 122.174) (width 0.25) (layer B.Cu) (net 7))
 (segment (start 184.817001 123.349001) (end 222.344999 123.349001) (width 0.25) (layer B.Cu) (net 7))
 (segment (start 183.642 122.174) (end 184.817001 123.349001) (width 0.25) (layer B.Cu) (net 7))
 (segment (start 182.277001 120.998999) (end 181.102 122.174) (width 0.25) (layer F.Cu) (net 8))
 (segment (start 219.804999 120.998999) (end 182.277001 120.998999) (width 0.25) (layer F.Cu) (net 8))
 (segment (start 220.98 122.174) (end 219.804999 120.998999) (width 0.25) (layer F.Cu) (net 8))
 (segment (start 184.817001 125.889001) (end 183.642 124.714) (width 0.25) (layer B.Cu) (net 5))
 (segment (start 222.344999 125.889001) (end 184.817001 125.889001) (width 0.25) (layer B.Cu) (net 5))
 (segment (start 223.52 124.714) (end 222.344999 125.889001) (width 0.25) (layer B.Cu) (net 5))
 (segment (start 181.102 124.714) (end 181.902998 124.714) (width 0.25) (layer F.Cu) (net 6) (status 30))
 (segment (start 219.804999 123.538999) (end 220.98 124.714) (width 0.25) (layer F.Cu) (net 6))
 (segment (start 182.277001 123.538999) (end 219.804999 123.538999) (width 0.25) (layer F.Cu) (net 6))
 (segment (start 181.102 124.714) (end 182.277001 123.538999) (width 0.25) (layer F.Cu) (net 6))
 (segment (start 222.344999 128.429001) (end 223.52 127.254) (width 0.25) (layer B.Cu) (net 3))
 (segment (start 184.817001 128.429001) (end 222.344999 128.429001) (width 0.25) (layer B.Cu) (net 3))
 (segment (start 183.642 127.254) (end 184.817001 128.429001) (width 0.25) (layer B.Cu) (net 3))
 (segment (start 182.277001 126.078999) (end 181.102 127.254) (width 0.25) (layer F.Cu) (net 4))
 (segment (start 219.804999 126.078999) (end 182.277001 126.078999) (width 0.25) (layer F.Cu) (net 4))
 (segment (start 220.98 127.254) (end 219.804999 126.078999) (width 0.25) (layer F.Cu) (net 4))
 (segment (start 222.344999 130.969001) (end 223.52 129.794) (width 0.25) (layer B.Cu) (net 1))
 (segment (start 184.817001 130.969001) (end 222.344999 130.969001) (width 0.25) (layer B.Cu) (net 1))
 (segment (start 183.642 129.794) (end 184.817001 130.969001) (width 0.25) (layer B.Cu) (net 1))
 (segment (start 219.804999 130.969001) (end 220.98 129.794) (width 0.25) (layer F.Cu) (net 2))
 (segment (start 182.277001 130.969001) (end 219.804999 130.969001) (width 0.25) (layer F.Cu) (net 2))
 (segment (start 181.102 129.794) (end 182.277001 130.969001) (width 0.25) (layer F.Cu) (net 2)))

